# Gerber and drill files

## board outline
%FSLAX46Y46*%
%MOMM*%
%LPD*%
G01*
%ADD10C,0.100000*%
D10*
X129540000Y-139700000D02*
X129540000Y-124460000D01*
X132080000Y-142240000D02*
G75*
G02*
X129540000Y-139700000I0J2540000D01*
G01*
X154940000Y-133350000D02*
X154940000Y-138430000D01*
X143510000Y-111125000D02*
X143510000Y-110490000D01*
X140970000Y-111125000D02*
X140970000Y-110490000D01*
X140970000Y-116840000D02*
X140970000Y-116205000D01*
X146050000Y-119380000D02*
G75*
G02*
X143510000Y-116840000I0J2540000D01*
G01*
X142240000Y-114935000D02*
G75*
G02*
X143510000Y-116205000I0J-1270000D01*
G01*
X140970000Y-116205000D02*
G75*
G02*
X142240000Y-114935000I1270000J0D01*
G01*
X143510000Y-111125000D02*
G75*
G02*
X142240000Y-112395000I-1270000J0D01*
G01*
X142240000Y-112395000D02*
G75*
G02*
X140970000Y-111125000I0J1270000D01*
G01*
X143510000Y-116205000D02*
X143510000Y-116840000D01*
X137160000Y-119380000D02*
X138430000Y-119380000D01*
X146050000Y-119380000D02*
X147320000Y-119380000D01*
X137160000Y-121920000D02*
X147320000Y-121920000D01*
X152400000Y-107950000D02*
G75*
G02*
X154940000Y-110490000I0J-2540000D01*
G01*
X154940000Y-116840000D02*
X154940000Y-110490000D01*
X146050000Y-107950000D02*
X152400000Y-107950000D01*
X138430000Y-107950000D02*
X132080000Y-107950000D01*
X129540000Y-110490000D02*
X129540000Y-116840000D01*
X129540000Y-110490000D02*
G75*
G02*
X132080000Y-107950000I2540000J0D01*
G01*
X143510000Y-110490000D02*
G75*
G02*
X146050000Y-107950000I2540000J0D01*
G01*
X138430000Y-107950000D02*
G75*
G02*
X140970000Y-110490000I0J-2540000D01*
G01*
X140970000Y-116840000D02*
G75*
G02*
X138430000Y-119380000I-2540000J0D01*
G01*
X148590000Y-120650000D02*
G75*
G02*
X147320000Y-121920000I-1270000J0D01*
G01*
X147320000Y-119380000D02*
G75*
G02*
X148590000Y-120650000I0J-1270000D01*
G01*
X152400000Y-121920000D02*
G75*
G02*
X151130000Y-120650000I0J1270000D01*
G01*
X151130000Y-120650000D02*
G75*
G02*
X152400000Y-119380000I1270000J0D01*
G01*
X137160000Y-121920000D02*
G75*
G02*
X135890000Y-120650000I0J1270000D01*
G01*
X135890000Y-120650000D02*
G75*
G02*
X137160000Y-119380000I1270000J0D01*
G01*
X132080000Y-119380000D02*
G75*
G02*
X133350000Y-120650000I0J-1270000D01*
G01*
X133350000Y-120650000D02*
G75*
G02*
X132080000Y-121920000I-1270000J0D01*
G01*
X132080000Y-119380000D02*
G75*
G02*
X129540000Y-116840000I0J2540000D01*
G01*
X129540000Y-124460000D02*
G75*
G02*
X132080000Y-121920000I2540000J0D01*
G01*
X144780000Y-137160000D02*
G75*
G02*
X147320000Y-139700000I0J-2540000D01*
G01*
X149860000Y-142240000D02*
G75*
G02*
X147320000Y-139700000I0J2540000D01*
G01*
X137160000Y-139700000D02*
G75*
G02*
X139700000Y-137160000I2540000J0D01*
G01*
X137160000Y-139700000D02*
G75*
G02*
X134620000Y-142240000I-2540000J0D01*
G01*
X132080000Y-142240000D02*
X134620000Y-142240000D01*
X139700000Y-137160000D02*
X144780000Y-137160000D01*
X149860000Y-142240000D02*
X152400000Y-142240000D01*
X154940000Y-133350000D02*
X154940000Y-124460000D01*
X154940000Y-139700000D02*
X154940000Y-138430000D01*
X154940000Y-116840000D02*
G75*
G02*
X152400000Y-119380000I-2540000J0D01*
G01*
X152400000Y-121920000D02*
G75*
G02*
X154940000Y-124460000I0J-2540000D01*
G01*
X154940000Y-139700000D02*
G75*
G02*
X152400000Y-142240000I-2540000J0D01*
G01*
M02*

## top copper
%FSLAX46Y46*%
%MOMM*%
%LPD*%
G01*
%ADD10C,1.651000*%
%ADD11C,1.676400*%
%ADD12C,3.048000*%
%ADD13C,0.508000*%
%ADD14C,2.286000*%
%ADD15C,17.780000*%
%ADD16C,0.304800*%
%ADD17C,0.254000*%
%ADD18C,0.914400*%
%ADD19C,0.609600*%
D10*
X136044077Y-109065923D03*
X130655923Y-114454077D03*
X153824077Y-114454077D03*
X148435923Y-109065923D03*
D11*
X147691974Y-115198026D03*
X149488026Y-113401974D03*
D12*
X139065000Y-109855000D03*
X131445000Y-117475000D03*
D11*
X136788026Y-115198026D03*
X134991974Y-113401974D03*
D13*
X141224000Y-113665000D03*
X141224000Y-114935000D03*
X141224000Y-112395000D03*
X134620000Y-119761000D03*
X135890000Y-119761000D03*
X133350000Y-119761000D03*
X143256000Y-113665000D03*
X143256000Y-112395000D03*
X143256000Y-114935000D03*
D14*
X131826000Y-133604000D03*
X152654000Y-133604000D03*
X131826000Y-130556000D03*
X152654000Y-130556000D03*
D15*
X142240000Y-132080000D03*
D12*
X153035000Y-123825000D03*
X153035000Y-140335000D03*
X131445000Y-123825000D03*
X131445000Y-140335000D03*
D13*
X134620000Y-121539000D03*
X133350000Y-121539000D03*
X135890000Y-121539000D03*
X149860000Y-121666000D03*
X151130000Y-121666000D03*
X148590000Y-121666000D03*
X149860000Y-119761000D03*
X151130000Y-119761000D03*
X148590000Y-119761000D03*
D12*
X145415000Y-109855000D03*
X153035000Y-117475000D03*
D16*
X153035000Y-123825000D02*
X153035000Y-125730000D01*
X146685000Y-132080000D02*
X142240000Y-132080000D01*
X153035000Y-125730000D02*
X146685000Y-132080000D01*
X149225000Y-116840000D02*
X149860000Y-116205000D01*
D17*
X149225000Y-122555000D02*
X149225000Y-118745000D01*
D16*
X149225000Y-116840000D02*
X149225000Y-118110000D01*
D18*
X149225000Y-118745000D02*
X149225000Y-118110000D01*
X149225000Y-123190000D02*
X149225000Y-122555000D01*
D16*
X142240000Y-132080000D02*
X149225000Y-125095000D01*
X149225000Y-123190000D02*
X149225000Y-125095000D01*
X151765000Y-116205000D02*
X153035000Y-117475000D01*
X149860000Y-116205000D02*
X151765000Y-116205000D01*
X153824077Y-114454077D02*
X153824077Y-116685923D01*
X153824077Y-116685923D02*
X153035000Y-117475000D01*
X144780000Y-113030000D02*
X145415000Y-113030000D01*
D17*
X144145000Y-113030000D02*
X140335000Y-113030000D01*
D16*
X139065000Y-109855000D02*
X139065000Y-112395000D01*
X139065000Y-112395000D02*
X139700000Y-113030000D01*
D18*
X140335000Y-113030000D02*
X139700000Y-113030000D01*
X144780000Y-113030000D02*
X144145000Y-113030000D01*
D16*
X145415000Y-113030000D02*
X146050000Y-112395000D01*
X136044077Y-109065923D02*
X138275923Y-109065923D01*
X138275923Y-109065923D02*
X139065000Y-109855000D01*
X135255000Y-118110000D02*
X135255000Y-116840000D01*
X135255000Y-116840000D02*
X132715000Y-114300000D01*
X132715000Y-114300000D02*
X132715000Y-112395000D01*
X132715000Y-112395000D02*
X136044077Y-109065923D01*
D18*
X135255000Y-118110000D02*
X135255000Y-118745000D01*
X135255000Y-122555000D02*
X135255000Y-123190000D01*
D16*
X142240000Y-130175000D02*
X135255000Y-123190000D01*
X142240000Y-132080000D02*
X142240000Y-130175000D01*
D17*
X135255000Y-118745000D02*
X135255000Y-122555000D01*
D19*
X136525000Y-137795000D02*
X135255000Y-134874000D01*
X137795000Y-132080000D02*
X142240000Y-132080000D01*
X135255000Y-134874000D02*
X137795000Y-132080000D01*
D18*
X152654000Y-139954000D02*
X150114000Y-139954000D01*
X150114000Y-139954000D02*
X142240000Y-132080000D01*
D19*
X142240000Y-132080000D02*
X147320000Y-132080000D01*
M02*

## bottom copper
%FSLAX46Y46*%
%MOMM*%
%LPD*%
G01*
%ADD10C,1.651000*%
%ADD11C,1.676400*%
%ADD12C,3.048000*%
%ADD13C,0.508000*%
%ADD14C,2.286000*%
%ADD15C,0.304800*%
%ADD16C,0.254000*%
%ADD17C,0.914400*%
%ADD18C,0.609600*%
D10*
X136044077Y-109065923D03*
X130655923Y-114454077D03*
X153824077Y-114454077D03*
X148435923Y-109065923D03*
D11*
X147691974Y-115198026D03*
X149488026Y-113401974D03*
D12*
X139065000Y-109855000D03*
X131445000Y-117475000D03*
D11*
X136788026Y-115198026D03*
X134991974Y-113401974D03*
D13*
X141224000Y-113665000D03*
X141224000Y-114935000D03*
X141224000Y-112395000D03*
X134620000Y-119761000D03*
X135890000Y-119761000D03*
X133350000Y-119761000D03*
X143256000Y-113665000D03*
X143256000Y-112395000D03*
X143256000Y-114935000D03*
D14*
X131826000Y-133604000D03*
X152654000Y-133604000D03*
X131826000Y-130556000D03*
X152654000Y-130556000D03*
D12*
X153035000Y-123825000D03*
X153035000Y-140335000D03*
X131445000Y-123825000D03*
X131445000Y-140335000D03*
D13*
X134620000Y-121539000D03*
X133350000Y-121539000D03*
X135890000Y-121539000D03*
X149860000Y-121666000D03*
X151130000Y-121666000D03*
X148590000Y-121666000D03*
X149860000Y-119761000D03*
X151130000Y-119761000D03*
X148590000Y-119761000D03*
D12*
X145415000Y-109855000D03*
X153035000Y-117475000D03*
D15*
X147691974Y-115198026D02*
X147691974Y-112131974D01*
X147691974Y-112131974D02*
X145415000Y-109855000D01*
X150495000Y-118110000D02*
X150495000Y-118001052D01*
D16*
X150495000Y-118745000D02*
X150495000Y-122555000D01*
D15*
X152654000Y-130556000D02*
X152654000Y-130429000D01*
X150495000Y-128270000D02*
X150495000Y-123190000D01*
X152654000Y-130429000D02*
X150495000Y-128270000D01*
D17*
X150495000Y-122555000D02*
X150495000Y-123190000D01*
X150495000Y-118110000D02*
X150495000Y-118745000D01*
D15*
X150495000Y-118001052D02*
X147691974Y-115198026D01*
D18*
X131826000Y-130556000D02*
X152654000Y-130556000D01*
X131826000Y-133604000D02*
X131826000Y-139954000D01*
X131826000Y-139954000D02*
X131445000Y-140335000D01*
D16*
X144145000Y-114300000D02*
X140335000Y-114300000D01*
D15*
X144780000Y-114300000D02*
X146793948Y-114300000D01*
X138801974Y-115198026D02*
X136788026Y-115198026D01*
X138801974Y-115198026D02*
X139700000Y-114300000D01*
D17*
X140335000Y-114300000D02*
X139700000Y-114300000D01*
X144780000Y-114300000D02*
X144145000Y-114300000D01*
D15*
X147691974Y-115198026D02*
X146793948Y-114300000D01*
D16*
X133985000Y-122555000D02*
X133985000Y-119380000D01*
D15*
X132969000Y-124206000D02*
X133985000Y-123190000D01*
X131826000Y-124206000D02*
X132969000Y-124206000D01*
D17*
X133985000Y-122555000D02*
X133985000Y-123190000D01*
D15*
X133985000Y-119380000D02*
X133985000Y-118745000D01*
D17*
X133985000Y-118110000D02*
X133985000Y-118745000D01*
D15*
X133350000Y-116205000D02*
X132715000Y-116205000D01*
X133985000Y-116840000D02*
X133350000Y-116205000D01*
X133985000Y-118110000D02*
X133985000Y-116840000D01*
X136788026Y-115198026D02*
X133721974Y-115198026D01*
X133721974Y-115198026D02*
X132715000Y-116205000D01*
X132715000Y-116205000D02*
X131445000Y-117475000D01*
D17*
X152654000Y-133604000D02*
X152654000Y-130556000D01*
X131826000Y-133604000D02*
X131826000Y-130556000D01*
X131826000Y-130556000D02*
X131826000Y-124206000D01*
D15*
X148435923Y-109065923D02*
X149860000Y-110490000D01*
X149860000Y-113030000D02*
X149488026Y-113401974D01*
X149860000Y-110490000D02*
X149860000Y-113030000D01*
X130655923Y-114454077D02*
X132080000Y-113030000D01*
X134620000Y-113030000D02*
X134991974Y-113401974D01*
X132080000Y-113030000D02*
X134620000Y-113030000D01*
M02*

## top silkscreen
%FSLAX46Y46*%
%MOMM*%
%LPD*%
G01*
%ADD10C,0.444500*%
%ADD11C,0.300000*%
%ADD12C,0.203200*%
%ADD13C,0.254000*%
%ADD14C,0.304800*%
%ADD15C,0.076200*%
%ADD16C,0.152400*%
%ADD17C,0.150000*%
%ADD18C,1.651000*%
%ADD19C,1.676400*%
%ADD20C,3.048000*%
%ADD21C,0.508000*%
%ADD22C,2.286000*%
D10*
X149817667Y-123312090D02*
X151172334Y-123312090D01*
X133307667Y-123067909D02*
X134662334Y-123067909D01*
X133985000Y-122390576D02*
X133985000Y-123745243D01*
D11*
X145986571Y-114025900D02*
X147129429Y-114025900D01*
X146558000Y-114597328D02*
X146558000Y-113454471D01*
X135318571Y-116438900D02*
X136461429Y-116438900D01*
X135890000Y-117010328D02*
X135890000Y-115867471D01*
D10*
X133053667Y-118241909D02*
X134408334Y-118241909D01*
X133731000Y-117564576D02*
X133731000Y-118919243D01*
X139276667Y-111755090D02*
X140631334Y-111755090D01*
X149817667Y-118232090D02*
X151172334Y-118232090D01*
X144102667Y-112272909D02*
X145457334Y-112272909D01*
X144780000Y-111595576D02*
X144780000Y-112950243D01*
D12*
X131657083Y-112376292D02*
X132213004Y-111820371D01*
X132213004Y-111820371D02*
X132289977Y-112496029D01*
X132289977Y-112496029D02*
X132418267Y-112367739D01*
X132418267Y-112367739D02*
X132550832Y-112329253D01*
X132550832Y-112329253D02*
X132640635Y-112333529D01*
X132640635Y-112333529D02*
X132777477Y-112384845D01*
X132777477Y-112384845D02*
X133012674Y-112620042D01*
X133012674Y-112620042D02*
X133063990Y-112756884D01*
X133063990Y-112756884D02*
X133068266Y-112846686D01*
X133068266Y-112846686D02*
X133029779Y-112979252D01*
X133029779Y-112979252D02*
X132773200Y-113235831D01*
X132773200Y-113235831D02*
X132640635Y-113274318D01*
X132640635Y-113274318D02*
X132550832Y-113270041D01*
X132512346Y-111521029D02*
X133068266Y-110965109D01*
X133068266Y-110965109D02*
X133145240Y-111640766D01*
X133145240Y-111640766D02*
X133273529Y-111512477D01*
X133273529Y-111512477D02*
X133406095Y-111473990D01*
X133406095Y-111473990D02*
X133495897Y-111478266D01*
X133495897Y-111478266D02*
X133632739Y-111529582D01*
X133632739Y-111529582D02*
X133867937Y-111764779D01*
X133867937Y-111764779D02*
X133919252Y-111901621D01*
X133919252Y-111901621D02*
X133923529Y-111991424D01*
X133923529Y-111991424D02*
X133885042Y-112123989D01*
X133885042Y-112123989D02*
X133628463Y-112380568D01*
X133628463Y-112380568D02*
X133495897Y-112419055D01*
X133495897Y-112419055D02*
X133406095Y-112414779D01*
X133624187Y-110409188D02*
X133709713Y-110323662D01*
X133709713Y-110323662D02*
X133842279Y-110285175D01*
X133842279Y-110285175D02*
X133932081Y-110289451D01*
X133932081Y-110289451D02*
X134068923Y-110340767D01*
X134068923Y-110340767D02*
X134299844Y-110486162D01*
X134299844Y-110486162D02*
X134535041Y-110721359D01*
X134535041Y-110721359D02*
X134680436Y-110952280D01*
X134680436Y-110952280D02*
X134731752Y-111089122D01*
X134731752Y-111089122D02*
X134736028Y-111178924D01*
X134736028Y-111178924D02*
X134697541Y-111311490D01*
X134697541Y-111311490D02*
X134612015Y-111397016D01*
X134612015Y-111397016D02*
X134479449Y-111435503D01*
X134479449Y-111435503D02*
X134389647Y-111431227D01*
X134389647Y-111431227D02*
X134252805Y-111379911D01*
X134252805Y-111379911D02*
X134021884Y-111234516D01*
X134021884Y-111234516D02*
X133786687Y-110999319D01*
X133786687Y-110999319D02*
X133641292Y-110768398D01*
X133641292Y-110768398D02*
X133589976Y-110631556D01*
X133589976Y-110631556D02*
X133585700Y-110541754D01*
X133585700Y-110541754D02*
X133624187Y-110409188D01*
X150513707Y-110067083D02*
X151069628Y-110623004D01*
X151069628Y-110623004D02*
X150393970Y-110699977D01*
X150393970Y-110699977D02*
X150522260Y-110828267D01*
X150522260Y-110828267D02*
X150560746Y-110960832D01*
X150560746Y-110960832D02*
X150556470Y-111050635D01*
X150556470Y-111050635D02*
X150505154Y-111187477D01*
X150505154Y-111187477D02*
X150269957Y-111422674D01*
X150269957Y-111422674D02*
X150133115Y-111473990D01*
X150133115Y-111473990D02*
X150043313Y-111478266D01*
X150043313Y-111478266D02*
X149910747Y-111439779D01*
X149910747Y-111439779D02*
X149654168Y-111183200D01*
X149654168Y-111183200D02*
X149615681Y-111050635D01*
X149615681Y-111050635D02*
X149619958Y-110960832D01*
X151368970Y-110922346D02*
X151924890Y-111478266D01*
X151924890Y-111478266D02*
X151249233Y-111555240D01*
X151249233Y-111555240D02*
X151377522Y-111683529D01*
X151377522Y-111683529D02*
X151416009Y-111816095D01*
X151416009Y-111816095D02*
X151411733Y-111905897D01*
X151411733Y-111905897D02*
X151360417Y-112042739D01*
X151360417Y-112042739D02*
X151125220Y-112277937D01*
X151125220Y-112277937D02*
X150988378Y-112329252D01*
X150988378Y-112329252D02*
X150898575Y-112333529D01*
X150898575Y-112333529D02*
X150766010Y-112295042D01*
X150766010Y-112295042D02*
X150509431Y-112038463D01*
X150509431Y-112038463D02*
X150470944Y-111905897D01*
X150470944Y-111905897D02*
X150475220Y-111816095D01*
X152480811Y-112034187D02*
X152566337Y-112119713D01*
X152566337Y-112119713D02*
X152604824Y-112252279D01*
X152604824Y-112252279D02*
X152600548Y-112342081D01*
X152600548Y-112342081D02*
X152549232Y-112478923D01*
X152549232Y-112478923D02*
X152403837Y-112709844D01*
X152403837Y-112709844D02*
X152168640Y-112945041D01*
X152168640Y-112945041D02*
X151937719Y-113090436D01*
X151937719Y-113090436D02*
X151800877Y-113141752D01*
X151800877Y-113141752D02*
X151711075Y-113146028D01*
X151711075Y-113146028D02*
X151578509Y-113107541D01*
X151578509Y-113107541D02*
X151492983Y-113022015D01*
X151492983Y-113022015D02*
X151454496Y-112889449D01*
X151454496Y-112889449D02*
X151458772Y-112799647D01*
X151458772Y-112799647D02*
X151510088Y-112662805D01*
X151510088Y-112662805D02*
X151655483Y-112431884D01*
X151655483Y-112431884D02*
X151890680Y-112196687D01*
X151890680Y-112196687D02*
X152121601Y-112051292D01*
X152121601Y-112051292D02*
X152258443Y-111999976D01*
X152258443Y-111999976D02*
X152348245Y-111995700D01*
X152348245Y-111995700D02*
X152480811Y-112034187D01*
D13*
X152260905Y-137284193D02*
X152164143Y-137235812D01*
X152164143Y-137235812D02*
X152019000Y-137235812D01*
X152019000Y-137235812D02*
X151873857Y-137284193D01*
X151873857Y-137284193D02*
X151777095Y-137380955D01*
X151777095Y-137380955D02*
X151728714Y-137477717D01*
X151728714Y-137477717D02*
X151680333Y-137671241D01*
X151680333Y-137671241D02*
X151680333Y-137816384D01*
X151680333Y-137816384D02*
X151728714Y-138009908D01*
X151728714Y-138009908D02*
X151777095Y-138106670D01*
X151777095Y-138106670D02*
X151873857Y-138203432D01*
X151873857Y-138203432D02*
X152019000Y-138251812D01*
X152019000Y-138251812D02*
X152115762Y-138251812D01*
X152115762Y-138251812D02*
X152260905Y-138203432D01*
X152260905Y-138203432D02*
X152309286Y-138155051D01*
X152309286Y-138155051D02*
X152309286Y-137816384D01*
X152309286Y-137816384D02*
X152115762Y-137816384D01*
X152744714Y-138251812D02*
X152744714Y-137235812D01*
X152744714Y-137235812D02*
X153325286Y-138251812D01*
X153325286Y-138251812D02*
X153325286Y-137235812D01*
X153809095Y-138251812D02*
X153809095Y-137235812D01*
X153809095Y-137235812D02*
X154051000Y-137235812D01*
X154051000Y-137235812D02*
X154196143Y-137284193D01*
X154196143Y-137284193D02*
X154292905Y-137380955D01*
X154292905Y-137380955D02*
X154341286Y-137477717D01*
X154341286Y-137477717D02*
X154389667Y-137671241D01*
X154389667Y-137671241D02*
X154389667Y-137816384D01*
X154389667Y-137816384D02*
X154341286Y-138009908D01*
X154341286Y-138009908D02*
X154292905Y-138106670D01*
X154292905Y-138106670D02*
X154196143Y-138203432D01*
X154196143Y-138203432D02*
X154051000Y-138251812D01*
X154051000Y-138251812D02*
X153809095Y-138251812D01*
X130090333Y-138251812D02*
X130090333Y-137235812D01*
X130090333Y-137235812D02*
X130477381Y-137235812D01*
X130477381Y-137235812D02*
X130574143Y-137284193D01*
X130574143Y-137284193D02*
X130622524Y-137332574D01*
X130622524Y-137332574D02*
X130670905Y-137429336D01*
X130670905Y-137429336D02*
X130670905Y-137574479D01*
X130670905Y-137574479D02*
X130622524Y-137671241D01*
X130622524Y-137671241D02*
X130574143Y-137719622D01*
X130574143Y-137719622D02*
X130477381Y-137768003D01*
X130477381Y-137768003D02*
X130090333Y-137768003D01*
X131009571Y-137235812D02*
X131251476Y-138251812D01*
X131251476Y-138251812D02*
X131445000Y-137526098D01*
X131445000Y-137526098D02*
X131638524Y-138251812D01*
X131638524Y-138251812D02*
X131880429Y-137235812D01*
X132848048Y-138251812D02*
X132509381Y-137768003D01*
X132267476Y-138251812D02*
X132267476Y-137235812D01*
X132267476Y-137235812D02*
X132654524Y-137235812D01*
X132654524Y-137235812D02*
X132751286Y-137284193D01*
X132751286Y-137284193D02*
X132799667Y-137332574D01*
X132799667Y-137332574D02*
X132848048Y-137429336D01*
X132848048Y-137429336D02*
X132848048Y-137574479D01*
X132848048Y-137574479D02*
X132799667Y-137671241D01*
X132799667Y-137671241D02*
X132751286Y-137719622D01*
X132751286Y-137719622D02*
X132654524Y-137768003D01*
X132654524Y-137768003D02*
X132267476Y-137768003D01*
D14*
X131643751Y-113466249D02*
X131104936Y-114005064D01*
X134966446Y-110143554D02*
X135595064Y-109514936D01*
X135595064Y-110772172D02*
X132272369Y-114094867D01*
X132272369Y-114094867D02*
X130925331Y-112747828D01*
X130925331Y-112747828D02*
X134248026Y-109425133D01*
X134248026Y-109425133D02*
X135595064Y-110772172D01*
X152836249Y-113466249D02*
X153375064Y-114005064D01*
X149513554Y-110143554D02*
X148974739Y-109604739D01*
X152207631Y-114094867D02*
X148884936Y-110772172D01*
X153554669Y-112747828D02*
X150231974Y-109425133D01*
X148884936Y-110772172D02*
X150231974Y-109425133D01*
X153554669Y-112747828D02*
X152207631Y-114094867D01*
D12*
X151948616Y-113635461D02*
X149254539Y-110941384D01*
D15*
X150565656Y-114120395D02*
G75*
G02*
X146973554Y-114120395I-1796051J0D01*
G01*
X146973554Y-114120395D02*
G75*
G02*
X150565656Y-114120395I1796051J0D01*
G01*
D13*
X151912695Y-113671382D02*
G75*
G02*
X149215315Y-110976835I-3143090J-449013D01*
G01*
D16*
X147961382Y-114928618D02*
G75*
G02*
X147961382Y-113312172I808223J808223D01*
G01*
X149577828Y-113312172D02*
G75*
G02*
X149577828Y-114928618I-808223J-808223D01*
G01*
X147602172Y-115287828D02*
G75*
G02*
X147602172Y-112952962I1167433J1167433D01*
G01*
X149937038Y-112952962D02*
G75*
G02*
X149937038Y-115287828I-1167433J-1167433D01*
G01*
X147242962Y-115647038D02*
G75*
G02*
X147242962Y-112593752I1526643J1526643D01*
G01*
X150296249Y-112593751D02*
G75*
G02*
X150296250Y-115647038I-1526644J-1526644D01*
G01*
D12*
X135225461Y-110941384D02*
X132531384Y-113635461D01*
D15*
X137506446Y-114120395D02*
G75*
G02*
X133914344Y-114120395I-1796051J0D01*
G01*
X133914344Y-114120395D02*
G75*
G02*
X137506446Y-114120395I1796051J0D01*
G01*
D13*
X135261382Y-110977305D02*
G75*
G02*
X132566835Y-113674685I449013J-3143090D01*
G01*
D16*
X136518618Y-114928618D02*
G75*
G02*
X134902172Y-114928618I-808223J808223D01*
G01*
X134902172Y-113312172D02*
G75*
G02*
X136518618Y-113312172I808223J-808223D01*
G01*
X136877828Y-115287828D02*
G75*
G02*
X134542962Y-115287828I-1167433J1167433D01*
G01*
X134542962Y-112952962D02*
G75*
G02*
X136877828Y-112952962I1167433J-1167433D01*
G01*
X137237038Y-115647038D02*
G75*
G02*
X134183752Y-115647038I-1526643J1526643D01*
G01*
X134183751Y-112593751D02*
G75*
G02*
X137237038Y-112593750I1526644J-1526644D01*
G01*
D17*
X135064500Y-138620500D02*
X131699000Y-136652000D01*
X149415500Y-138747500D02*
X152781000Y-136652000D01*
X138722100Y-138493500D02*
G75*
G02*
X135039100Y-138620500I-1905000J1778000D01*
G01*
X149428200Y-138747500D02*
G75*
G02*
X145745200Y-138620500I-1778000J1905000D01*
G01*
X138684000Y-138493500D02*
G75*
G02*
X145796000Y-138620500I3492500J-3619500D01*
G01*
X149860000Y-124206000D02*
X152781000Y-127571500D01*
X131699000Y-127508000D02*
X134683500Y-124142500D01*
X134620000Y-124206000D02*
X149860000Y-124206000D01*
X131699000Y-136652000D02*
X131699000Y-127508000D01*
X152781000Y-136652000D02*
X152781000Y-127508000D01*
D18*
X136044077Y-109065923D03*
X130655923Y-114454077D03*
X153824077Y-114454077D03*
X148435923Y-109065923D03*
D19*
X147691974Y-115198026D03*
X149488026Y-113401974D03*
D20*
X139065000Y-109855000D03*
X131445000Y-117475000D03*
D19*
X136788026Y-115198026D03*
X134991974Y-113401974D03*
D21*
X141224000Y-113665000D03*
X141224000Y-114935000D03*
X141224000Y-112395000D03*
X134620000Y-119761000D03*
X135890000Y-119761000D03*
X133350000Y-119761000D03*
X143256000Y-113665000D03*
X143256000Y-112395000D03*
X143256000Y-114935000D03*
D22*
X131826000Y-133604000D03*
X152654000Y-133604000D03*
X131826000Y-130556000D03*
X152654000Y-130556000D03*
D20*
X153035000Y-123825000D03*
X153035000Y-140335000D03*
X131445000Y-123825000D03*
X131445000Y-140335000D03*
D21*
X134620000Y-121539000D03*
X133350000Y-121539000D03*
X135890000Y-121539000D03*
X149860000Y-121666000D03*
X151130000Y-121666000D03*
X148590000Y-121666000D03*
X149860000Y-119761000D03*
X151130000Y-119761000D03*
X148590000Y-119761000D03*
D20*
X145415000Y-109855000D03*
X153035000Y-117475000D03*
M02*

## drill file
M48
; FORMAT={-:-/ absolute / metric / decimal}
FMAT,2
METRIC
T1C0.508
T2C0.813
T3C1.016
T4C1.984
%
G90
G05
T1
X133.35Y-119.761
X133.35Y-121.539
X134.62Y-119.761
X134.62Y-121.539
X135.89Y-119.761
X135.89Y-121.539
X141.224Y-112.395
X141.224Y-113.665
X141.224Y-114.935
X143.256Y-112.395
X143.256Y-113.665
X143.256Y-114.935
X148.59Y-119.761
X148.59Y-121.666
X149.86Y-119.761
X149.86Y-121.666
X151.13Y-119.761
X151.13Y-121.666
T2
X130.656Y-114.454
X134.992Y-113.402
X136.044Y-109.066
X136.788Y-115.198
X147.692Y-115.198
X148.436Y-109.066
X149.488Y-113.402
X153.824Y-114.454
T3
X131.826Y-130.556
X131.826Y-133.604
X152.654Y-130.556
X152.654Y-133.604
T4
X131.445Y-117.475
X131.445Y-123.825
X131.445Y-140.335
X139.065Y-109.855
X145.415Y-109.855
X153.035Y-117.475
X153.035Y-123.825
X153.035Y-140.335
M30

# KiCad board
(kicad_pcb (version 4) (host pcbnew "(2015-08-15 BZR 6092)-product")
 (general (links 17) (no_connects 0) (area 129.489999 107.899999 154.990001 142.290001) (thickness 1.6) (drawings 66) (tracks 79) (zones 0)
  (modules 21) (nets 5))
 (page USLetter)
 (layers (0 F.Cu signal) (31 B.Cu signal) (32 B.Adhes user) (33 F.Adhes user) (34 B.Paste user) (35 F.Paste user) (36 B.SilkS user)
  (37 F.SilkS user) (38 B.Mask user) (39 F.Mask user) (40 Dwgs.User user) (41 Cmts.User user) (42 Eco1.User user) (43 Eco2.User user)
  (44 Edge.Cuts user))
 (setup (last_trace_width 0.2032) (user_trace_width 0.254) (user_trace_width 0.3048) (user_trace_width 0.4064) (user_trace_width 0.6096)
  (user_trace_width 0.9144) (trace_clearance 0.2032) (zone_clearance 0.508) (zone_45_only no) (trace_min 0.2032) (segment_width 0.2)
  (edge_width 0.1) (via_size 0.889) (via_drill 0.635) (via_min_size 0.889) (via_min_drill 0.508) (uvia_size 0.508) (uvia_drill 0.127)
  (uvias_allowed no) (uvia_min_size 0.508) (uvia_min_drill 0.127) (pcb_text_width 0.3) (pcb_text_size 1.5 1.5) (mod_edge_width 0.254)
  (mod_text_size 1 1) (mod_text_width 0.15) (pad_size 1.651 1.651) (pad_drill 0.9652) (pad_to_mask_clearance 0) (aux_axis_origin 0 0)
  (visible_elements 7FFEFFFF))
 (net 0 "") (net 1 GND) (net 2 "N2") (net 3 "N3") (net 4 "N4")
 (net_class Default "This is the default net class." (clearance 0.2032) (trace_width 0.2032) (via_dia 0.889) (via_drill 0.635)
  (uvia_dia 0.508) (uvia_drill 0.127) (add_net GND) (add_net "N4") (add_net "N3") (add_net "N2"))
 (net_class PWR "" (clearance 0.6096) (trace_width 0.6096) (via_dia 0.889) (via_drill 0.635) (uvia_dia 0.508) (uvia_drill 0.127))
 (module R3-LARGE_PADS (layer F.Cu) (at 133.35 111.76 225) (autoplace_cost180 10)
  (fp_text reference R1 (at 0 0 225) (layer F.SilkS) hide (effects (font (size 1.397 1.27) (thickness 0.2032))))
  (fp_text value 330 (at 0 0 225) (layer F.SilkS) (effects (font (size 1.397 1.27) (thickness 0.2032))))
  (fp_line (start 2.413 0) (end 3.175 0) (layer F.SilkS) (width 0.3048))
  (fp_line (start -2.286 0) (end -3.175 0) (layer F.SilkS) (width 0.3048))
  (fp_line (start -2.286 -0.889) (end 2.413 -0.889) (layer F.SilkS) (width 0.3048))
  (fp_line (start 2.413 -0.889) (end 2.413 1.016) (layer F.SilkS) (width 0.3048))
  (fp_line (start 2.413 1.016) (end -2.286 1.016) (layer F.SilkS) (width 0.3048))
  (fp_line (start -2.286 1.016) (end -2.286 -0.889) (layer F.SilkS) (width 0.3048))
  (pad 1 thru_hole circle (at -3.81 0 225) (size 1.651 1.651) (drill 0.8128) (layers *.Cu *.Mask F.SilkS) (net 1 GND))
  (pad 2 thru_hole circle (at 3.81 0 225) (size 1.651 1.651) (drill 0.8128) (layers *.Cu *.Mask F.SilkS) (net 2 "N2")))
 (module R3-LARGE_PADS (layer F.Cu) (at 151.13 111.76 135) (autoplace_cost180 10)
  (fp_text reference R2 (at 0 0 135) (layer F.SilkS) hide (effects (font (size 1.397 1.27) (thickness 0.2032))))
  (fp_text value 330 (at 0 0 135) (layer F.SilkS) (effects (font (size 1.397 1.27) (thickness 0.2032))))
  (fp_line (start -2.413 0) (end -3.175 0) (layer F.SilkS) (width 0.3048))
  (fp_line (start 2.286 0) (end 3.048 0) (layer F.SilkS) (width 0.3048))
  (fp_line (start -2.413 -0.889) (end 2.286 -0.889) (layer F.SilkS) (width 0.3048))
  (fp_line (start -2.413 1.016) (end 2.286 1.016) (layer F.SilkS) (width 0.3048))
  (fp_line (start 2.286 -0.889) (end 2.286 1.016) (layer F.SilkS) (width 0.3048))
  (fp_line (start -2.413 1.016) (end -2.413 -0.889) (layer F.SilkS) (width 0.3048))
  (pad 1 thru_hole circle (at -3.81 0 135) (size 1.651 1.651) (drill 0.8128) (layers *.Cu *.Mask F.SilkS) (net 1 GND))
  (pad 2 thru_hole circle (at 3.81 0 135) (size 1.651 1.651) (drill 0.8128) (layers *.Cu *.Mask F.SilkS) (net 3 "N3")))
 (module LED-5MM (layer F.Cu) (at 148.59 114.3 45)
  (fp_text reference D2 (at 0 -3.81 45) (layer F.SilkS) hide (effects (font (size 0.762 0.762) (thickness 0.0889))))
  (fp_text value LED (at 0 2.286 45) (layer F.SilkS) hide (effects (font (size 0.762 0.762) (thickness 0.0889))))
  (fp_line (start 2.8448 1.905) (end 2.8448 -1.905) (layer F.SilkS) (width 0.2032))
  (fp_circle (center 0.254 0) (end -1.016 1.27) (layer F.SilkS) (width 0.0762))
  (fp_arc (start 0.254 0) (end 2.794 1.905) (angle 286.2) (layer F.SilkS) (width 0.254))
  (fp_arc (start 0.254 0) (end -0.889 0) (angle 90) (layer F.SilkS) (width 0.1524))
  (fp_arc (start 0.254 0) (end 1.397 0) (angle 90) (layer F.SilkS) (width 0.1524))
  (fp_arc (start 0.254 0) (end -1.397 0) (angle 90) (layer F.SilkS) (width 0.1524))
  (fp_arc (start 0.254 0) (end 1.905 0) (angle 90) (layer F.SilkS) (width 0.1524))
  (fp_arc (start 0.254 0) (end -1.905 0) (angle 90) (layer F.SilkS) (width 0.1524))
  (fp_arc (start 0.254 0) (end 2.413 0) (angle 90) (layer F.SilkS) (width 0.1524))
  (pad 1 thru_hole circle (at -1.27 0 45) (size 1.6764 1.6764) (drill 0.8128) (layers *.Cu *.Mask F.SilkS) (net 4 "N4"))
  (pad 2 thru_hole circle (at 1.27 0 45) (size 1.6764 1.6764) (drill 0.8128) (layers *.Cu *.Mask F.SilkS) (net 3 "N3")))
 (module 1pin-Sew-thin (layer F.Cu) (at 139.065 109.855 270)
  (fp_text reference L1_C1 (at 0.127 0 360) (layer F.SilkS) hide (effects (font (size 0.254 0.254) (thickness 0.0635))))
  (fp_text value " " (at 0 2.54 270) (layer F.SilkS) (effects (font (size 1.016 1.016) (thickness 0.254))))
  (pad 1 thru_hole circle (at 0 0 270) (size 3.048 3.048) (drill 1.984375) (layers *.Cu *.Mask F.SilkS) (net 1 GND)))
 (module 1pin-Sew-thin (layer F.Cu) (at 131.445 117.475 270)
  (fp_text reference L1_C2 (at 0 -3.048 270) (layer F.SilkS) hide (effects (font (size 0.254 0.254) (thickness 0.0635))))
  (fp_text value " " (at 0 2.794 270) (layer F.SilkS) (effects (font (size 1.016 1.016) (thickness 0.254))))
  (pad 1 thru_hole circle (at 0 0 270) (size 3.048 3.048) (drill 1.984375) (layers *.Cu *.Mask F.SilkS) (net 4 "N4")))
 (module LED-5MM (layer F.Cu) (at 135.89 114.3 135)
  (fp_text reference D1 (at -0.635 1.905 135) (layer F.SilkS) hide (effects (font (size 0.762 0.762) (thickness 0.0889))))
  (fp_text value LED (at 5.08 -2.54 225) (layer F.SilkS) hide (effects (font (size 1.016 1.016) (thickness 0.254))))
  (fp_line (start 2.8448 1.905) (end 2.8448 -1.905) (layer F.SilkS) (width 0.2032))
  (fp_circle (center 0.254 0) (end -1.016 1.27) (layer F.SilkS) (width 0.0762))
  (fp_arc (start 0.254 0) (end 2.794 1.905) (angle 286.2) (layer F.SilkS) (width 0.254))
  (fp_arc (start 0.254 0) (end -0.889 0) (angle 90) (layer F.SilkS) (width 0.1524))
  (fp_arc (start 0.254 0) (end 1.397 0) (angle 90) (layer F.SilkS) (width 0.1524))
  (fp_arc (start 0.254 0) (end -1.397 0) (angle 90) (layer F.SilkS) (width 0.1524))
  (fp_arc (start 0.254 0) (end 1.905 0) (angle 90) (layer F.SilkS) (width 0.1524))
  (fp_arc (start 0.254 0) (end -1.905 0) (angle 90) (layer F.SilkS) (width 0.1524))
  (fp_arc (start 0.254 0) (end 2.413 0) (angle 90) (layer F.SilkS) (width 0.1524))
  (pad 1 thru_hole circle (at -1.27 0 135) (size 1.6764 1.6764) (drill 0.8128) (layers *.Cu *.Mask F.SilkS) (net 4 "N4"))
  (pad 2 thru_hole circle (at 1.27 0 135) (size 1.6764 1.6764) (drill 0.8128) (layers *.Cu *.Mask F.SilkS) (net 2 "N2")))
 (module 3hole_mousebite (layer F.Cu) (at 141.605 113.665 90)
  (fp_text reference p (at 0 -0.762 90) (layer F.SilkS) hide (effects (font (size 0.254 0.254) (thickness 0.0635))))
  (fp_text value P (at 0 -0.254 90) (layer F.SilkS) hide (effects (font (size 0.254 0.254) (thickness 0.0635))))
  (pad "" thru_hole circle (at 0 -0.381 90) (size 0.508 0.508) (drill 0.508) (layers *.Cu *.Mask F.SilkS))
  (pad 1 thru_hole circle (at -1.27 -0.381 90) (size 0.508 0.508) (drill 0.508) (layers *.Cu *.Mask F.SilkS))
  (pad 2 thru_hole circle (at 1.27 -0.381 90) (size 0.508 0.508) (drill 0.508) (layers *.Cu *.Mask F.SilkS)))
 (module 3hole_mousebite (layer F.Cu) (at 134.62 119.38 180)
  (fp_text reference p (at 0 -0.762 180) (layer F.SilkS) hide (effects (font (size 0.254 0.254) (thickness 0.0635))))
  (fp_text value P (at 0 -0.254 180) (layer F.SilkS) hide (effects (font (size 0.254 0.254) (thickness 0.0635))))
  (pad "" thru_hole circle (at 0 -0.381 180) (size 0.508 0.508) (drill 0.508) (layers *.Cu *.Mask F.SilkS))
  (pad 1 thru_hole circle (at -1.27 -0.381 180) (size 0.508 0.508) (drill 0.508) (layers *.Cu *.Mask F.SilkS))
  (pad 2 thru_hole circle (at 1.27 -0.381 180) (size 0.508 0.508) (drill 0.508) (layers *.Cu *.Mask F.SilkS)))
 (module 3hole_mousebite (layer F.Cu) (at 142.875 113.665 270)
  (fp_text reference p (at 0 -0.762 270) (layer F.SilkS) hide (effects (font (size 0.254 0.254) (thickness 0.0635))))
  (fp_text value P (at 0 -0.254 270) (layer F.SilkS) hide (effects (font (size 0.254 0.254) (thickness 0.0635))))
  (pad "" thru_hole circle (at 0 -0.381 270) (size 0.508 0.508) (drill 0.508) (layers *.Cu *.Mask F.SilkS))
  (pad 1 thru_hole circle (at -1.27 -0.381 270) (size 0.508 0.508) (drill 0.508) (layers *.Cu *.Mask F.SilkS))
  (pad 2 thru_hole circle (at 1.27 -0.381 270) (size 0.508 0.508) (drill 0.508) (layers *.Cu *.Mask F.SilkS)))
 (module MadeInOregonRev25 (layer F.Cu) (at 137.033 131.699)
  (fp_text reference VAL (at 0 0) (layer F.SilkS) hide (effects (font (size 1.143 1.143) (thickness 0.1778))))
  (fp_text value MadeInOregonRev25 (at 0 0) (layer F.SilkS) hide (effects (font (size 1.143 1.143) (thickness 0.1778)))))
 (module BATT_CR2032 (layer F.Cu) (at 142.24 132.08)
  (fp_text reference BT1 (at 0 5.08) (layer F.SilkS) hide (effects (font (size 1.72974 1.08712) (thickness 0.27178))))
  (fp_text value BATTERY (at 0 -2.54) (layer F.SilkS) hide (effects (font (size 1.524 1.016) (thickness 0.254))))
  (fp_line (start -7.1755 6.5405) (end -10.541 4.572) (layer F.SilkS) (width 0.15))
  (fp_line (start 7.1755 6.6675) (end 10.541 4.572) (layer F.SilkS) (width 0.15))
  (fp_arc (start -5.4229 4.6355) (end -3.5179 6.4135) (angle 90) (layer F.SilkS) (width 0.15))
  (fp_arc (start 5.4102 4.7625) (end 7.1882 6.6675) (angle 90) (layer F.SilkS) (width 0.15))
  (fp_arc (start -0.0635 10.033) (end -3.556 6.4135) (angle 90) (layer F.SilkS) (width 0.15))
  (fp_line (start 7.62 -7.874) (end 10.541 -4.5085) (layer F.SilkS) (width 0.15))
  (fp_line (start -10.541 -4.572) (end -7.5565 -7.9375) (layer F.SilkS) (width 0.15))
  (fp_line (start -7.62 -7.874) (end 7.62 -7.874) (layer F.SilkS) (width 0.15))
  (fp_line (start -10.541 4.572) (end -10.541 -4.572) (layer F.SilkS) (width 0.15))
  (fp_line (start 10.541 4.572) (end 10.541 -4.572) (layer F.SilkS) (width 0.15))
  (pad 1 thru_hole circle (at -10.414 1.524) (size 2.286 2.286) (drill 1.016) (layers *.Cu *.Mask F.SilkS) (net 4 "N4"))
  (pad 1 thru_hole circle (at 10.414 1.524) (size 2.286 2.286) (drill 1.016) (layers *.Cu *.Mask F.SilkS) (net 4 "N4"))
  (pad 1 thru_hole circle (at -10.414 -1.524) (size 2.286 2.286) (drill 1.016) (layers *.Cu *.Mask F.SilkS) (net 4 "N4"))
  (pad 1 thru_hole circle (at 10.414 -1.524) (size 2.286 2.286) (drill 1.016) (layers *.Cu *.Mask F.SilkS) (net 4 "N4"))
  (pad 2 smd circle (at 0 0) (size 17.78 17.78) (layers F.Cu F.Paste F.Mask) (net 1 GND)))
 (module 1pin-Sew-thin (layer F.Cu) (at 153.035 123.825)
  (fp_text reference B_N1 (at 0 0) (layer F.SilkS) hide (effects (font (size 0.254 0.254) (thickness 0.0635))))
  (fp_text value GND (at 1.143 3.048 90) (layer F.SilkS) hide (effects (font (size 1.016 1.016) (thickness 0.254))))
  (pad 1 thru_hole circle (at 0 0) (size 3.048 3.048) (drill 1.984375) (layers *.Cu *.Mask F.SilkS) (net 1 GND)))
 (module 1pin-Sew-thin (layer F.Cu) (at 153.035 140.335)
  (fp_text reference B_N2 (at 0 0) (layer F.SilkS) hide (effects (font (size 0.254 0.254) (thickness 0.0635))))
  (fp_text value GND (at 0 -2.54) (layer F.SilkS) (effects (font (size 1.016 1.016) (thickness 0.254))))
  (pad 1 thru_hole circle (at 0 0) (size 3.048 3.048) (drill 1.984375) (layers *.Cu *.Mask F.SilkS) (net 1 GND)))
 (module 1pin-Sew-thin (layer F.Cu) (at 131.445 123.825)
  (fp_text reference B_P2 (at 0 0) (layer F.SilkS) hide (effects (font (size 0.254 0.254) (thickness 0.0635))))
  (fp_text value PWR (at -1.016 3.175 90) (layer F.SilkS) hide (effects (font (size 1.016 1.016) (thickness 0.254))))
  (pad 1 thru_hole circle (at 0 0) (size 3.048 3.048) (drill 1.984375) (layers *.Cu *.Mask F.SilkS) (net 4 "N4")))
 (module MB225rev (layer F.Cu) (at 147.447 131.699)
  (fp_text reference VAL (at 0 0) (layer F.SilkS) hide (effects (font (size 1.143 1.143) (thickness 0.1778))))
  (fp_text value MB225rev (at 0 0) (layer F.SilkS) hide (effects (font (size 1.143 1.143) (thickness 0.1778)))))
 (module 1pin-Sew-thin (layer F.Cu) (at 131.445 140.335)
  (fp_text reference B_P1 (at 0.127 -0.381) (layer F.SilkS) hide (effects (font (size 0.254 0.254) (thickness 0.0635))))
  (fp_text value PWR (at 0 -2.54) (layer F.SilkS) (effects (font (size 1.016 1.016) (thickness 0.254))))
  (pad 1 thru_hole circle (at 0 0) (size 3.048 3.048) (drill 1.984375) (layers *.Cu *.Mask F.SilkS) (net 4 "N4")))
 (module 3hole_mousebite (layer F.Cu) (at 134.62 121.92)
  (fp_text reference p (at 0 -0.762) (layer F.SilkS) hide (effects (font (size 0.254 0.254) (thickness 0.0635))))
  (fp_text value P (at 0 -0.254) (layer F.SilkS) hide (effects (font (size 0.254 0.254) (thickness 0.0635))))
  (pad "" thru_hole circle (at 0 -0.381) (size 0.508 0.508) (drill 0.508) (layers *.Cu *.Mask F.SilkS))
  (pad 1 thru_hole circle (at -1.27 -0.381) (size 0.508 0.508) (drill 0.508) (layers *.Cu *.Mask F.SilkS))
  (pad 2 thru_hole circle (at 1.27 -0.381) (size 0.508 0.508) (drill 0.508) (layers *.Cu *.Mask F.SilkS)))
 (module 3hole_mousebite (layer F.Cu) (at 149.86 121.285 180)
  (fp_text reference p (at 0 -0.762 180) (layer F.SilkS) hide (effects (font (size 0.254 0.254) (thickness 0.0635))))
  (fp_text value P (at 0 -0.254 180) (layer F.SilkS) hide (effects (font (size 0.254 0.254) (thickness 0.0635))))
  (pad "" thru_hole circle (at 0 -0.381 180) (size 0.508 0.508) (drill 0.508) (layers *.Cu *.Mask F.SilkS))
  (pad 1 thru_hole circle (at -1.27 -0.381 180) (size 0.508 0.508) (drill 0.508) (layers *.Cu *.Mask F.SilkS))
  (pad 2 thru_hole circle (at 1.27 -0.381 180) (size 0.508 0.508) (drill 0.508) (layers *.Cu *.Mask F.SilkS)))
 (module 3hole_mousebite (layer F.Cu) (at 149.86 119.38 180)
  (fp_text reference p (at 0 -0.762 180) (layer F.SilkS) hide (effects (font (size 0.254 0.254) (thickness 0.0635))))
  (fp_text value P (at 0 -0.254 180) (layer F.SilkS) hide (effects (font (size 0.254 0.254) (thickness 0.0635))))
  (pad "" thru_hole circle (at 0 -0.381 180) (size 0.508 0.508) (drill 0.508) (layers *.Cu *.Mask F.SilkS))
  (pad 1 thru_hole circle (at -1.27 -0.381 180) (size 0.508 0.508) (drill 0.508) (layers *.Cu *.Mask F.SilkS))
  (pad 2 thru_hole circle (at 1.27 -0.381 180) (size 0.508 0.508) (drill 0.508) (layers *.Cu *.Mask F.SilkS)))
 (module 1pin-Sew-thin (layer F.Cu) (at 145.415 109.855)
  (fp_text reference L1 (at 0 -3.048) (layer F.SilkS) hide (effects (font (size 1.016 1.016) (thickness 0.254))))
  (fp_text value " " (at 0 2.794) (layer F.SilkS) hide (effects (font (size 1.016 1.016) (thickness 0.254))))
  (pad 1 thru_hole circle (at 0 0) (size 3.048 3.048) (drill 1.984375) (layers *.Cu *.Mask F.SilkS) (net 4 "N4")))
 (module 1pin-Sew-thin (layer F.Cu) (at 153.035 117.475)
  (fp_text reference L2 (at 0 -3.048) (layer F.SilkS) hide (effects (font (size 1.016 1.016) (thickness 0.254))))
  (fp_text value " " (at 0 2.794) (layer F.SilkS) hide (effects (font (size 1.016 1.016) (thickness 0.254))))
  (pad 1 thru_hole circle (at 0 0) (size 3.048 3.048) (drill 1.984375) (layers *.Cu *.Mask F.SilkS) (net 1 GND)))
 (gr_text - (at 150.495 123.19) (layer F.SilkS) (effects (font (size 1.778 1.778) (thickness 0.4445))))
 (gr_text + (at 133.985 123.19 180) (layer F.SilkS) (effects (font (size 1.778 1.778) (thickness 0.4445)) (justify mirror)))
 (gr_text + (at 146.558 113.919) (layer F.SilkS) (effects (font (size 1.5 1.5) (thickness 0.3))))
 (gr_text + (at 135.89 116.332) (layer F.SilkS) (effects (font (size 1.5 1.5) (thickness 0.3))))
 (gr_line (start 129.54 139.7) (end 129.54 124.46) (angle 90) (layer Edge.Cuts) (width 0.1))
 (gr_arc (start 132.08 139.7) (end 132.08 142.24) (angle 90) (layer Edge.Cuts) (width 0.1))
 (gr_line (start 154.94 133.35) (end 154.94 138.43) (angle 90) (layer Edge.Cuts) (width 0.1))
 (gr_line (start 143.51 111.125) (end 143.51 110.49) (angle 90) (layer Edge.Cuts) (width 0.1))
 (gr_line (start 140.97 111.125) (end 140.97 110.49) (angle 90) (layer Edge.Cuts) (width 0.1))
 (gr_line (start 140.97 116.84) (end 140.97 116.205) (angle 90) (layer Edge.Cuts) (width 0.1))
 (gr_arc (start 146.05 116.84) (end 146.05 119.38) (angle 90) (layer Edge.Cuts) (width 0.1))
 (gr_arc (start 142.24 116.205) (end 142.24 114.935) (angle 90) (layer Edge.Cuts) (width 0.1))
 (gr_arc (start 142.24 116.205) (end 140.97 116.205) (angle 90) (layer Edge.Cuts) (width 0.1))
 (gr_arc (start 142.24 111.125) (end 143.51 111.125) (angle 90) (layer Edge.Cuts) (width 0.1))
 (gr_arc (start 142.24 111.125) (end 142.24 112.395) (angle 90) (layer Edge.Cuts) (width 0.1))
 (gr_line (start 143.51 116.205) (end 143.51 116.84) (angle 90) (layer Edge.Cuts) (width 0.1))
 (gr_line (start 137.16 119.38) (end 138.43 119.38) (angle 90) (layer Edge.Cuts) (width 0.1))
 (gr_line (start 146.05 119.38) (end 147.32 119.38) (angle 90) (layer Edge.Cuts) (width 0.1))
 (gr_line (start 137.16 121.92) (end 147.32 121.92) (angle 90) (layer Edge.Cuts) (width 0.1))
 (gr_arc (start 152.4 110.49) (end 152.4 107.95) (angle 90) (layer Edge.Cuts) (width 0.1))
 (gr_line (start 154.94 116.84) (end 154.94 110.49) (angle 90) (layer Edge.Cuts) (width 0.1))
 (gr_line (start 146.05 107.95) (end 152.4 107.95) (angle 90) (layer Edge.Cuts) (width 0.1))
 (gr_line (start 138.43 107.95) (end 132.08 107.95) (angle 90) (layer Edge.Cuts) (width 0.1))
 (gr_line (start 129.54 110.49) (end 129.54 116.84) (angle 90) (layer Edge.Cuts) (width 0.1))
 (gr_arc (start 132.08 110.49) (end 129.54 110.49) (angle 90) (layer Edge.Cuts) (width 0.1))
 (gr_arc (start 146.05 110.49) (end 143.51 110.49) (angle 90) (layer Edge.Cuts) (width 0.1))
 (gr_arc (start 138.43 110.49) (end 138.43 107.95) (angle 90) (layer Edge.Cuts) (width 0.1))
 (gr_arc (start 138.43 116.84) (end 140.97 116.84) (angle 90) (layer Edge.Cuts) (width 0.1))
 (gr_arc (start 147.32 120.65) (end 148.59 120.65) (angle 90) (layer Edge.Cuts) (width 0.1))
 (gr_arc (start 147.32 120.65) (end 147.32 119.38) (angle 90) (layer Edge.Cuts) (width 0.1))
 (gr_arc (start 152.4 120.65) (end 152.4 121.92) (angle 90) (layer Edge.Cuts) (width 0.1))
 (gr_arc (start 152.4 120.65) (end 151.13 120.65) (angle 90) (layer Edge.Cuts) (width 0.1))
 (gr_arc (start 137.16 120.65) (end 137.16 121.92) (angle 90) (layer Edge.Cuts) (width 0.1))
 (gr_arc (start 137.16 120.65) (end 135.89 120.65) (angle 90) (layer Edge.Cuts) (width 0.1))
 (gr_arc (start 132.08 120.65) (end 132.08 119.38) (angle 90) (layer Edge.Cuts) (width 0.1))
 (gr_arc (start 132.08 120.65) (end 133.35 120.65) (angle 90) (layer Edge.Cuts) (width 0.1))
 (gr_arc (start 132.08 116.84) (end 132.08 119.38) (angle 90) (layer Edge.Cuts) (width 0.1))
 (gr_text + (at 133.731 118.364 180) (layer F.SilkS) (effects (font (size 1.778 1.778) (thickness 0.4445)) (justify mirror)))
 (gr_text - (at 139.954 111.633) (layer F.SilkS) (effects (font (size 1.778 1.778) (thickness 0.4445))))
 (gr_arc (start 132.08 124.46) (end 129.54 124.46) (angle 90) (layer Edge.Cuts) (width 0.1))
 (gr_arc (start 144.78 139.7) (end 144.78 137.16) (angle 90) (layer Edge.Cuts) (width 0.1))
 (gr_arc (start 149.86 139.7) (end 149.86 142.24) (angle 90) (layer Edge.Cuts) (width 0.1))
 (gr_arc (start 139.7 139.7) (end 137.16 139.7) (angle 90) (layer Edge.Cuts) (width 0.1))
 (gr_arc (start 134.62 139.7) (end 137.16 139.7) (angle 90) (layer Edge.Cuts) (width 0.1))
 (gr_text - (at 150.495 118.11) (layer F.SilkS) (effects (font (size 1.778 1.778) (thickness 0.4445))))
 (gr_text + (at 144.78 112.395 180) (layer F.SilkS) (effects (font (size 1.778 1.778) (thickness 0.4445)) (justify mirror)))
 (gr_line (start 132.08 142.24) (end 134.62 142.24) (angle 90) (layer Edge.Cuts) (width 0.1))
 (gr_line (start 139.7 137.16) (end 144.78 137.16) (angle 90) (layer Edge.Cuts) (width 0.1))
 (gr_line (start 149.86 142.24) (end 152.4 142.24) (angle 90) (layer Edge.Cuts) (width 0.1))
 (gr_line (start 154.94 133.35) (end 154.94 124.46) (angle 90) (layer Edge.Cuts) (width 0.1))
 (gr_line (start 154.94 139.7) (end 154.94 138.43) (angle 90) (layer Edge.Cuts) (width 0.1))
 (gr_arc (start 152.4 116.84) (end 154.94 116.84) (angle 90) (layer Edge.Cuts) (width 0.1))
 (gr_arc (start 152.4 124.46) (end 152.4 121.92) (angle 90) (layer Edge.Cuts) (width 0.1))
 (gr_arc (start 152.4 139.7) (end 154.94 139.7) (angle 90) (layer Edge.Cuts) (width 0.1))
 (segment (start 153.035 123.825) (end 153.035 125.73) (width 0.3048) (layer F.Cu) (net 1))
 (segment (start 146.685 132.08) (end 142.24 132.08) (width 0.3048) (layer F.Cu) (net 1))
 (segment (start 153.035 125.73) (end 146.685 132.08) (width 0.3048) (layer F.Cu) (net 1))
 (segment (start 149.225 116.84) (end 149.86 116.205) (width 0.3048) (layer F.Cu) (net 1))
 (segment (start 149.225 122.555) (end 149.225 118.745) (width 0.254) (layer F.Cu) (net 1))
 (segment (start 149.225 116.84) (end 149.225 118.11) (width 0.3048) (layer F.Cu) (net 1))
 (segment (start 149.225 118.745) (end 149.225 118.11) (width 0.9144) (layer F.Cu) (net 1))
 (segment (start 149.225 123.19) (end 149.225 122.555) (width 0.9144) (layer F.Cu) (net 1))
 (segment (start 142.24 132.08) (end 149.225 125.095) (width 0.3048) (layer F.Cu) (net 1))
 (segment (start 149.225 123.19) (end 149.225 125.095) (width 0.3048) (layer F.Cu) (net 1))
 (segment (start 151.765 116.205) (end 153.035 117.475) (width 0.3048) (layer F.Cu) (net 1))
 (segment (start 149.86 116.205) (end 151.765 116.205) (width 0.3048) (layer F.Cu) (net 1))
 (segment (start 153.824077 114.454077) (end 153.824077 116.685923) (width 0.3048) (layer F.Cu) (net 1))
 (segment (start 153.824077 116.685923) (end 153.035 117.475) (width 0.3048) (layer F.Cu) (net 1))
 (segment (start 144.78 113.03) (end 145.415 113.03) (width 0.3048) (layer F.Cu) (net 1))
 (segment (start 144.145 113.03) (end 140.335 113.03) (width 0.254) (layer F.Cu) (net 1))
 (segment (start 139.065 109.855) (end 139.065 112.395) (width 0.3048) (layer F.Cu) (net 1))
 (segment (start 139.065 112.395) (end 139.7 113.03) (width 0.3048) (layer F.Cu) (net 1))
 (segment (start 140.335 113.03) (end 139.7 113.03) (width 0.9144) (layer F.Cu) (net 1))
 (segment (start 144.78 113.03) (end 144.145 113.03) (width 0.9144) (layer F.Cu) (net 1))
 (segment (start 145.415 113.03) (end 146.05 112.395) (width 0.3048) (layer F.Cu) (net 1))
 (segment (start 136.044077 109.065923) (end 138.275923 109.065923) (width 0.3048) (layer F.Cu) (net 1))
 (segment (start 138.275923 109.065923) (end 139.065 109.855) (width 0.3048) (layer F.Cu) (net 1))
 (segment (start 135.255 118.11) (end 135.255 116.84) (width 0.3048) (layer F.Cu) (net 1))
 (segment (start 135.255 116.84) (end 132.715 114.3) (width 0.3048) (layer F.Cu) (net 1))
 (segment (start 132.715 114.3) (end 132.715 112.395) (width 0.3048) (layer F.Cu) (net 1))
 (segment (start 132.715 112.395) (end 136.044077 109.065923) (width 0.3048) (layer F.Cu) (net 1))
 (segment (start 135.255 118.11) (end 135.255 118.745) (width 0.9144) (layer F.Cu) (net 1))
 (segment (start 135.255 122.555) (end 135.255 123.19) (width 0.9144) (layer F.Cu) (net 1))
 (segment (start 142.24 130.175) (end 135.255 123.19) (width 0.3048) (layer F.Cu) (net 1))
 (segment (start 142.24 132.08) (end 142.24 130.175) (width 0.3048) (layer F.Cu) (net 1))
 (segment (start 135.255 118.745) (end 135.255 122.555) (width 0.254) (layer F.Cu) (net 1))
 (segment (start 136.525 137.795) (end 135.255 134.874) (width 0.6096) (layer F.Cu) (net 1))
 (segment (start 137.795 132.08) (end 142.24 132.08) (width 0.6096) (layer F.Cu) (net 1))
 (segment (start 135.255 134.874) (end 137.795 132.08) (width 0.6096) (layer F.Cu) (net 1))
 (segment (start 152.654 139.954) (end 150.114 139.954) (width 0.9144) (layer F.Cu) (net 1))
 (segment (start 150.114 139.954) (end 142.24 132.08) (width 0.9144) (layer F.Cu) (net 1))
 (segment (start 142.24 132.08) (end 147.32 132.08) (width 0.6096) (layer F.Cu) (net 1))
 (segment (start 147.691974 115.198026) (end 147.691974 112.131974) (width 0.3048) (layer B.Cu) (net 4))
 (segment (start 147.691974 112.131974) (end 145.415 109.855) (width 0.3048) (layer B.Cu) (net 4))
 (segment (start 150.495 118.11) (end 150.495 118.001052) (width 0.3048) (layer B.Cu) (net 4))
 (segment (start 150.495 118.745) (end 150.495 122.555) (width 0.254) (layer B.Cu) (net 4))
 (segment (start 152.654 130.556) (end 152.654 130.429) (width 0.3048) (layer B.Cu) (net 4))
 (segment (start 150.495 128.27) (end 150.495 123.19) (width 0.3048) (layer B.Cu) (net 4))
 (segment (start 152.654 130.429) (end 150.495 128.27) (width 0.3048) (layer B.Cu) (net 4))
 (segment (start 150.495 122.555) (end 150.495 123.19) (width 0.9144) (layer B.Cu) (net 4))
 (segment (start 150.495 118.11) (end 150.495 118.745) (width 0.9144) (layer B.Cu) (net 4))
 (segment (start 150.495 118.001052) (end 147.691974 115.198026) (width 0.3048) (layer B.Cu) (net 4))
 (segment (start 131.826 130.556) (end 152.654 130.556) (width 0.6096) (layer B.Cu) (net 4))
 (segment (start 131.826 133.604) (end 131.826 139.954) (width 0.6096) (layer B.Cu) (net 4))
 (segment (start 131.826 139.954) (end 131.445 140.335) (width 0.6096) (layer B.Cu) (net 4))
 (segment (start 144.145 114.3) (end 140.335 114.3) (width 0.254) (layer B.Cu) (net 4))
 (segment (start 144.78 114.3) (end 146.793948 114.3) (width 0.3048) (layer B.Cu) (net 4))
 (segment (start 138.801974 115.198026) (end 136.788026 115.198026) (width 0.3048) (layer B.Cu) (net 4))
 (segment (start 138.801974 115.198026) (end 139.7 114.3) (width 0.3048) (layer B.Cu) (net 4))
 (segment (start 140.335 114.3) (end 139.7 114.3) (width 0.9144) (layer B.Cu) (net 4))
 (segment (start 144.78 114.3) (end 144.145 114.3) (width 0.9144) (layer B.Cu) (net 4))
 (segment (start 147.691974 115.198026) (end 146.793948 114.3) (width 0.3048) (layer B.Cu) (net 4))
 (segment (start 133.985 122.555) (end 133.985 119.38) (width 0.254) (layer B.Cu) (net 4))
 (segment (start 132.969 124.206) (end 133.985 123.19) (width 0.3048) (layer B.Cu) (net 4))
 (segment (start 131.826 124.206) (end 132.969 124.206) (width 0.3048) (layer B.Cu) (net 4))
 (segment (start 133.985 122.555) (end 133.985 123.19) (width 0.9144) (layer B.Cu) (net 4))
 (segment (start 133.985 119.38) (end 133.985 118.745) (width 0.3048) (layer B.Cu) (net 4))
 (segment (start 133.985 118.11) (end 133.985 118.745) (width 0.9144) (layer B.Cu) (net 4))
 (segment (start 133.35 116.205) (end 132.715 116.205) (width 0.3048) (layer B.Cu) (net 4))
 (segment (start 133.985 116.84) (end 133.35 116.205) (width 0.3048) (layer B.Cu) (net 4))
 (segment (start 133.985 118.11) (end 133.985 116.84) (width 0.3048) (layer B.Cu) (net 4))
 (segment (start 136.788026 115.198026) (end 133.721974 115.198026) (width 0.3048) (layer B.Cu) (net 4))
 (segment (start 133.721974 115.198026) (end 132.715 116.205) (width 0.3048) (layer B.Cu) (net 4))
 (segment (start 132.715 116.205) (end 131.445 117.475) (width 0.3048) (layer B.Cu) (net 4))
 (segment (start 152.654 133.604) (end 152.654 130.556) (width 0.9144) (layer B.Cu) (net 4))
 (segment (start 131.826 133.604) (end 131.826 130.556) (width 0.9144) (layer B.Cu) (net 4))
 (segment (start 131.826 130.556) (end 131.826 124.206) (width 0.9144) (layer B.Cu) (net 4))
 (segment (start 148.435923 109.065923) (end 149.86 110.49) (width 0.3048) (layer B.Cu) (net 3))
 (segment (start 149.86 113.03) (end 149.488026 113.401974) (width 0.3048) (layer B.Cu) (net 3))
 (segment (start 149.86 110.49) (end 149.86 113.03) (width 0.3048) (layer B.Cu) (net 3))
 (segment (start 130.655923 114.454077) (end 132.08 113.03) (width 0.3048) (layer B.Cu) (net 2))
 (segment (start 134.62 113.03) (end 134.991974 113.401974) (width 0.3048) (layer B.Cu) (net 2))
 (segment (start 132.08 113.03) (end 134.62 113.03) (width 0.3048) (layer B.Cu) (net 2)))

